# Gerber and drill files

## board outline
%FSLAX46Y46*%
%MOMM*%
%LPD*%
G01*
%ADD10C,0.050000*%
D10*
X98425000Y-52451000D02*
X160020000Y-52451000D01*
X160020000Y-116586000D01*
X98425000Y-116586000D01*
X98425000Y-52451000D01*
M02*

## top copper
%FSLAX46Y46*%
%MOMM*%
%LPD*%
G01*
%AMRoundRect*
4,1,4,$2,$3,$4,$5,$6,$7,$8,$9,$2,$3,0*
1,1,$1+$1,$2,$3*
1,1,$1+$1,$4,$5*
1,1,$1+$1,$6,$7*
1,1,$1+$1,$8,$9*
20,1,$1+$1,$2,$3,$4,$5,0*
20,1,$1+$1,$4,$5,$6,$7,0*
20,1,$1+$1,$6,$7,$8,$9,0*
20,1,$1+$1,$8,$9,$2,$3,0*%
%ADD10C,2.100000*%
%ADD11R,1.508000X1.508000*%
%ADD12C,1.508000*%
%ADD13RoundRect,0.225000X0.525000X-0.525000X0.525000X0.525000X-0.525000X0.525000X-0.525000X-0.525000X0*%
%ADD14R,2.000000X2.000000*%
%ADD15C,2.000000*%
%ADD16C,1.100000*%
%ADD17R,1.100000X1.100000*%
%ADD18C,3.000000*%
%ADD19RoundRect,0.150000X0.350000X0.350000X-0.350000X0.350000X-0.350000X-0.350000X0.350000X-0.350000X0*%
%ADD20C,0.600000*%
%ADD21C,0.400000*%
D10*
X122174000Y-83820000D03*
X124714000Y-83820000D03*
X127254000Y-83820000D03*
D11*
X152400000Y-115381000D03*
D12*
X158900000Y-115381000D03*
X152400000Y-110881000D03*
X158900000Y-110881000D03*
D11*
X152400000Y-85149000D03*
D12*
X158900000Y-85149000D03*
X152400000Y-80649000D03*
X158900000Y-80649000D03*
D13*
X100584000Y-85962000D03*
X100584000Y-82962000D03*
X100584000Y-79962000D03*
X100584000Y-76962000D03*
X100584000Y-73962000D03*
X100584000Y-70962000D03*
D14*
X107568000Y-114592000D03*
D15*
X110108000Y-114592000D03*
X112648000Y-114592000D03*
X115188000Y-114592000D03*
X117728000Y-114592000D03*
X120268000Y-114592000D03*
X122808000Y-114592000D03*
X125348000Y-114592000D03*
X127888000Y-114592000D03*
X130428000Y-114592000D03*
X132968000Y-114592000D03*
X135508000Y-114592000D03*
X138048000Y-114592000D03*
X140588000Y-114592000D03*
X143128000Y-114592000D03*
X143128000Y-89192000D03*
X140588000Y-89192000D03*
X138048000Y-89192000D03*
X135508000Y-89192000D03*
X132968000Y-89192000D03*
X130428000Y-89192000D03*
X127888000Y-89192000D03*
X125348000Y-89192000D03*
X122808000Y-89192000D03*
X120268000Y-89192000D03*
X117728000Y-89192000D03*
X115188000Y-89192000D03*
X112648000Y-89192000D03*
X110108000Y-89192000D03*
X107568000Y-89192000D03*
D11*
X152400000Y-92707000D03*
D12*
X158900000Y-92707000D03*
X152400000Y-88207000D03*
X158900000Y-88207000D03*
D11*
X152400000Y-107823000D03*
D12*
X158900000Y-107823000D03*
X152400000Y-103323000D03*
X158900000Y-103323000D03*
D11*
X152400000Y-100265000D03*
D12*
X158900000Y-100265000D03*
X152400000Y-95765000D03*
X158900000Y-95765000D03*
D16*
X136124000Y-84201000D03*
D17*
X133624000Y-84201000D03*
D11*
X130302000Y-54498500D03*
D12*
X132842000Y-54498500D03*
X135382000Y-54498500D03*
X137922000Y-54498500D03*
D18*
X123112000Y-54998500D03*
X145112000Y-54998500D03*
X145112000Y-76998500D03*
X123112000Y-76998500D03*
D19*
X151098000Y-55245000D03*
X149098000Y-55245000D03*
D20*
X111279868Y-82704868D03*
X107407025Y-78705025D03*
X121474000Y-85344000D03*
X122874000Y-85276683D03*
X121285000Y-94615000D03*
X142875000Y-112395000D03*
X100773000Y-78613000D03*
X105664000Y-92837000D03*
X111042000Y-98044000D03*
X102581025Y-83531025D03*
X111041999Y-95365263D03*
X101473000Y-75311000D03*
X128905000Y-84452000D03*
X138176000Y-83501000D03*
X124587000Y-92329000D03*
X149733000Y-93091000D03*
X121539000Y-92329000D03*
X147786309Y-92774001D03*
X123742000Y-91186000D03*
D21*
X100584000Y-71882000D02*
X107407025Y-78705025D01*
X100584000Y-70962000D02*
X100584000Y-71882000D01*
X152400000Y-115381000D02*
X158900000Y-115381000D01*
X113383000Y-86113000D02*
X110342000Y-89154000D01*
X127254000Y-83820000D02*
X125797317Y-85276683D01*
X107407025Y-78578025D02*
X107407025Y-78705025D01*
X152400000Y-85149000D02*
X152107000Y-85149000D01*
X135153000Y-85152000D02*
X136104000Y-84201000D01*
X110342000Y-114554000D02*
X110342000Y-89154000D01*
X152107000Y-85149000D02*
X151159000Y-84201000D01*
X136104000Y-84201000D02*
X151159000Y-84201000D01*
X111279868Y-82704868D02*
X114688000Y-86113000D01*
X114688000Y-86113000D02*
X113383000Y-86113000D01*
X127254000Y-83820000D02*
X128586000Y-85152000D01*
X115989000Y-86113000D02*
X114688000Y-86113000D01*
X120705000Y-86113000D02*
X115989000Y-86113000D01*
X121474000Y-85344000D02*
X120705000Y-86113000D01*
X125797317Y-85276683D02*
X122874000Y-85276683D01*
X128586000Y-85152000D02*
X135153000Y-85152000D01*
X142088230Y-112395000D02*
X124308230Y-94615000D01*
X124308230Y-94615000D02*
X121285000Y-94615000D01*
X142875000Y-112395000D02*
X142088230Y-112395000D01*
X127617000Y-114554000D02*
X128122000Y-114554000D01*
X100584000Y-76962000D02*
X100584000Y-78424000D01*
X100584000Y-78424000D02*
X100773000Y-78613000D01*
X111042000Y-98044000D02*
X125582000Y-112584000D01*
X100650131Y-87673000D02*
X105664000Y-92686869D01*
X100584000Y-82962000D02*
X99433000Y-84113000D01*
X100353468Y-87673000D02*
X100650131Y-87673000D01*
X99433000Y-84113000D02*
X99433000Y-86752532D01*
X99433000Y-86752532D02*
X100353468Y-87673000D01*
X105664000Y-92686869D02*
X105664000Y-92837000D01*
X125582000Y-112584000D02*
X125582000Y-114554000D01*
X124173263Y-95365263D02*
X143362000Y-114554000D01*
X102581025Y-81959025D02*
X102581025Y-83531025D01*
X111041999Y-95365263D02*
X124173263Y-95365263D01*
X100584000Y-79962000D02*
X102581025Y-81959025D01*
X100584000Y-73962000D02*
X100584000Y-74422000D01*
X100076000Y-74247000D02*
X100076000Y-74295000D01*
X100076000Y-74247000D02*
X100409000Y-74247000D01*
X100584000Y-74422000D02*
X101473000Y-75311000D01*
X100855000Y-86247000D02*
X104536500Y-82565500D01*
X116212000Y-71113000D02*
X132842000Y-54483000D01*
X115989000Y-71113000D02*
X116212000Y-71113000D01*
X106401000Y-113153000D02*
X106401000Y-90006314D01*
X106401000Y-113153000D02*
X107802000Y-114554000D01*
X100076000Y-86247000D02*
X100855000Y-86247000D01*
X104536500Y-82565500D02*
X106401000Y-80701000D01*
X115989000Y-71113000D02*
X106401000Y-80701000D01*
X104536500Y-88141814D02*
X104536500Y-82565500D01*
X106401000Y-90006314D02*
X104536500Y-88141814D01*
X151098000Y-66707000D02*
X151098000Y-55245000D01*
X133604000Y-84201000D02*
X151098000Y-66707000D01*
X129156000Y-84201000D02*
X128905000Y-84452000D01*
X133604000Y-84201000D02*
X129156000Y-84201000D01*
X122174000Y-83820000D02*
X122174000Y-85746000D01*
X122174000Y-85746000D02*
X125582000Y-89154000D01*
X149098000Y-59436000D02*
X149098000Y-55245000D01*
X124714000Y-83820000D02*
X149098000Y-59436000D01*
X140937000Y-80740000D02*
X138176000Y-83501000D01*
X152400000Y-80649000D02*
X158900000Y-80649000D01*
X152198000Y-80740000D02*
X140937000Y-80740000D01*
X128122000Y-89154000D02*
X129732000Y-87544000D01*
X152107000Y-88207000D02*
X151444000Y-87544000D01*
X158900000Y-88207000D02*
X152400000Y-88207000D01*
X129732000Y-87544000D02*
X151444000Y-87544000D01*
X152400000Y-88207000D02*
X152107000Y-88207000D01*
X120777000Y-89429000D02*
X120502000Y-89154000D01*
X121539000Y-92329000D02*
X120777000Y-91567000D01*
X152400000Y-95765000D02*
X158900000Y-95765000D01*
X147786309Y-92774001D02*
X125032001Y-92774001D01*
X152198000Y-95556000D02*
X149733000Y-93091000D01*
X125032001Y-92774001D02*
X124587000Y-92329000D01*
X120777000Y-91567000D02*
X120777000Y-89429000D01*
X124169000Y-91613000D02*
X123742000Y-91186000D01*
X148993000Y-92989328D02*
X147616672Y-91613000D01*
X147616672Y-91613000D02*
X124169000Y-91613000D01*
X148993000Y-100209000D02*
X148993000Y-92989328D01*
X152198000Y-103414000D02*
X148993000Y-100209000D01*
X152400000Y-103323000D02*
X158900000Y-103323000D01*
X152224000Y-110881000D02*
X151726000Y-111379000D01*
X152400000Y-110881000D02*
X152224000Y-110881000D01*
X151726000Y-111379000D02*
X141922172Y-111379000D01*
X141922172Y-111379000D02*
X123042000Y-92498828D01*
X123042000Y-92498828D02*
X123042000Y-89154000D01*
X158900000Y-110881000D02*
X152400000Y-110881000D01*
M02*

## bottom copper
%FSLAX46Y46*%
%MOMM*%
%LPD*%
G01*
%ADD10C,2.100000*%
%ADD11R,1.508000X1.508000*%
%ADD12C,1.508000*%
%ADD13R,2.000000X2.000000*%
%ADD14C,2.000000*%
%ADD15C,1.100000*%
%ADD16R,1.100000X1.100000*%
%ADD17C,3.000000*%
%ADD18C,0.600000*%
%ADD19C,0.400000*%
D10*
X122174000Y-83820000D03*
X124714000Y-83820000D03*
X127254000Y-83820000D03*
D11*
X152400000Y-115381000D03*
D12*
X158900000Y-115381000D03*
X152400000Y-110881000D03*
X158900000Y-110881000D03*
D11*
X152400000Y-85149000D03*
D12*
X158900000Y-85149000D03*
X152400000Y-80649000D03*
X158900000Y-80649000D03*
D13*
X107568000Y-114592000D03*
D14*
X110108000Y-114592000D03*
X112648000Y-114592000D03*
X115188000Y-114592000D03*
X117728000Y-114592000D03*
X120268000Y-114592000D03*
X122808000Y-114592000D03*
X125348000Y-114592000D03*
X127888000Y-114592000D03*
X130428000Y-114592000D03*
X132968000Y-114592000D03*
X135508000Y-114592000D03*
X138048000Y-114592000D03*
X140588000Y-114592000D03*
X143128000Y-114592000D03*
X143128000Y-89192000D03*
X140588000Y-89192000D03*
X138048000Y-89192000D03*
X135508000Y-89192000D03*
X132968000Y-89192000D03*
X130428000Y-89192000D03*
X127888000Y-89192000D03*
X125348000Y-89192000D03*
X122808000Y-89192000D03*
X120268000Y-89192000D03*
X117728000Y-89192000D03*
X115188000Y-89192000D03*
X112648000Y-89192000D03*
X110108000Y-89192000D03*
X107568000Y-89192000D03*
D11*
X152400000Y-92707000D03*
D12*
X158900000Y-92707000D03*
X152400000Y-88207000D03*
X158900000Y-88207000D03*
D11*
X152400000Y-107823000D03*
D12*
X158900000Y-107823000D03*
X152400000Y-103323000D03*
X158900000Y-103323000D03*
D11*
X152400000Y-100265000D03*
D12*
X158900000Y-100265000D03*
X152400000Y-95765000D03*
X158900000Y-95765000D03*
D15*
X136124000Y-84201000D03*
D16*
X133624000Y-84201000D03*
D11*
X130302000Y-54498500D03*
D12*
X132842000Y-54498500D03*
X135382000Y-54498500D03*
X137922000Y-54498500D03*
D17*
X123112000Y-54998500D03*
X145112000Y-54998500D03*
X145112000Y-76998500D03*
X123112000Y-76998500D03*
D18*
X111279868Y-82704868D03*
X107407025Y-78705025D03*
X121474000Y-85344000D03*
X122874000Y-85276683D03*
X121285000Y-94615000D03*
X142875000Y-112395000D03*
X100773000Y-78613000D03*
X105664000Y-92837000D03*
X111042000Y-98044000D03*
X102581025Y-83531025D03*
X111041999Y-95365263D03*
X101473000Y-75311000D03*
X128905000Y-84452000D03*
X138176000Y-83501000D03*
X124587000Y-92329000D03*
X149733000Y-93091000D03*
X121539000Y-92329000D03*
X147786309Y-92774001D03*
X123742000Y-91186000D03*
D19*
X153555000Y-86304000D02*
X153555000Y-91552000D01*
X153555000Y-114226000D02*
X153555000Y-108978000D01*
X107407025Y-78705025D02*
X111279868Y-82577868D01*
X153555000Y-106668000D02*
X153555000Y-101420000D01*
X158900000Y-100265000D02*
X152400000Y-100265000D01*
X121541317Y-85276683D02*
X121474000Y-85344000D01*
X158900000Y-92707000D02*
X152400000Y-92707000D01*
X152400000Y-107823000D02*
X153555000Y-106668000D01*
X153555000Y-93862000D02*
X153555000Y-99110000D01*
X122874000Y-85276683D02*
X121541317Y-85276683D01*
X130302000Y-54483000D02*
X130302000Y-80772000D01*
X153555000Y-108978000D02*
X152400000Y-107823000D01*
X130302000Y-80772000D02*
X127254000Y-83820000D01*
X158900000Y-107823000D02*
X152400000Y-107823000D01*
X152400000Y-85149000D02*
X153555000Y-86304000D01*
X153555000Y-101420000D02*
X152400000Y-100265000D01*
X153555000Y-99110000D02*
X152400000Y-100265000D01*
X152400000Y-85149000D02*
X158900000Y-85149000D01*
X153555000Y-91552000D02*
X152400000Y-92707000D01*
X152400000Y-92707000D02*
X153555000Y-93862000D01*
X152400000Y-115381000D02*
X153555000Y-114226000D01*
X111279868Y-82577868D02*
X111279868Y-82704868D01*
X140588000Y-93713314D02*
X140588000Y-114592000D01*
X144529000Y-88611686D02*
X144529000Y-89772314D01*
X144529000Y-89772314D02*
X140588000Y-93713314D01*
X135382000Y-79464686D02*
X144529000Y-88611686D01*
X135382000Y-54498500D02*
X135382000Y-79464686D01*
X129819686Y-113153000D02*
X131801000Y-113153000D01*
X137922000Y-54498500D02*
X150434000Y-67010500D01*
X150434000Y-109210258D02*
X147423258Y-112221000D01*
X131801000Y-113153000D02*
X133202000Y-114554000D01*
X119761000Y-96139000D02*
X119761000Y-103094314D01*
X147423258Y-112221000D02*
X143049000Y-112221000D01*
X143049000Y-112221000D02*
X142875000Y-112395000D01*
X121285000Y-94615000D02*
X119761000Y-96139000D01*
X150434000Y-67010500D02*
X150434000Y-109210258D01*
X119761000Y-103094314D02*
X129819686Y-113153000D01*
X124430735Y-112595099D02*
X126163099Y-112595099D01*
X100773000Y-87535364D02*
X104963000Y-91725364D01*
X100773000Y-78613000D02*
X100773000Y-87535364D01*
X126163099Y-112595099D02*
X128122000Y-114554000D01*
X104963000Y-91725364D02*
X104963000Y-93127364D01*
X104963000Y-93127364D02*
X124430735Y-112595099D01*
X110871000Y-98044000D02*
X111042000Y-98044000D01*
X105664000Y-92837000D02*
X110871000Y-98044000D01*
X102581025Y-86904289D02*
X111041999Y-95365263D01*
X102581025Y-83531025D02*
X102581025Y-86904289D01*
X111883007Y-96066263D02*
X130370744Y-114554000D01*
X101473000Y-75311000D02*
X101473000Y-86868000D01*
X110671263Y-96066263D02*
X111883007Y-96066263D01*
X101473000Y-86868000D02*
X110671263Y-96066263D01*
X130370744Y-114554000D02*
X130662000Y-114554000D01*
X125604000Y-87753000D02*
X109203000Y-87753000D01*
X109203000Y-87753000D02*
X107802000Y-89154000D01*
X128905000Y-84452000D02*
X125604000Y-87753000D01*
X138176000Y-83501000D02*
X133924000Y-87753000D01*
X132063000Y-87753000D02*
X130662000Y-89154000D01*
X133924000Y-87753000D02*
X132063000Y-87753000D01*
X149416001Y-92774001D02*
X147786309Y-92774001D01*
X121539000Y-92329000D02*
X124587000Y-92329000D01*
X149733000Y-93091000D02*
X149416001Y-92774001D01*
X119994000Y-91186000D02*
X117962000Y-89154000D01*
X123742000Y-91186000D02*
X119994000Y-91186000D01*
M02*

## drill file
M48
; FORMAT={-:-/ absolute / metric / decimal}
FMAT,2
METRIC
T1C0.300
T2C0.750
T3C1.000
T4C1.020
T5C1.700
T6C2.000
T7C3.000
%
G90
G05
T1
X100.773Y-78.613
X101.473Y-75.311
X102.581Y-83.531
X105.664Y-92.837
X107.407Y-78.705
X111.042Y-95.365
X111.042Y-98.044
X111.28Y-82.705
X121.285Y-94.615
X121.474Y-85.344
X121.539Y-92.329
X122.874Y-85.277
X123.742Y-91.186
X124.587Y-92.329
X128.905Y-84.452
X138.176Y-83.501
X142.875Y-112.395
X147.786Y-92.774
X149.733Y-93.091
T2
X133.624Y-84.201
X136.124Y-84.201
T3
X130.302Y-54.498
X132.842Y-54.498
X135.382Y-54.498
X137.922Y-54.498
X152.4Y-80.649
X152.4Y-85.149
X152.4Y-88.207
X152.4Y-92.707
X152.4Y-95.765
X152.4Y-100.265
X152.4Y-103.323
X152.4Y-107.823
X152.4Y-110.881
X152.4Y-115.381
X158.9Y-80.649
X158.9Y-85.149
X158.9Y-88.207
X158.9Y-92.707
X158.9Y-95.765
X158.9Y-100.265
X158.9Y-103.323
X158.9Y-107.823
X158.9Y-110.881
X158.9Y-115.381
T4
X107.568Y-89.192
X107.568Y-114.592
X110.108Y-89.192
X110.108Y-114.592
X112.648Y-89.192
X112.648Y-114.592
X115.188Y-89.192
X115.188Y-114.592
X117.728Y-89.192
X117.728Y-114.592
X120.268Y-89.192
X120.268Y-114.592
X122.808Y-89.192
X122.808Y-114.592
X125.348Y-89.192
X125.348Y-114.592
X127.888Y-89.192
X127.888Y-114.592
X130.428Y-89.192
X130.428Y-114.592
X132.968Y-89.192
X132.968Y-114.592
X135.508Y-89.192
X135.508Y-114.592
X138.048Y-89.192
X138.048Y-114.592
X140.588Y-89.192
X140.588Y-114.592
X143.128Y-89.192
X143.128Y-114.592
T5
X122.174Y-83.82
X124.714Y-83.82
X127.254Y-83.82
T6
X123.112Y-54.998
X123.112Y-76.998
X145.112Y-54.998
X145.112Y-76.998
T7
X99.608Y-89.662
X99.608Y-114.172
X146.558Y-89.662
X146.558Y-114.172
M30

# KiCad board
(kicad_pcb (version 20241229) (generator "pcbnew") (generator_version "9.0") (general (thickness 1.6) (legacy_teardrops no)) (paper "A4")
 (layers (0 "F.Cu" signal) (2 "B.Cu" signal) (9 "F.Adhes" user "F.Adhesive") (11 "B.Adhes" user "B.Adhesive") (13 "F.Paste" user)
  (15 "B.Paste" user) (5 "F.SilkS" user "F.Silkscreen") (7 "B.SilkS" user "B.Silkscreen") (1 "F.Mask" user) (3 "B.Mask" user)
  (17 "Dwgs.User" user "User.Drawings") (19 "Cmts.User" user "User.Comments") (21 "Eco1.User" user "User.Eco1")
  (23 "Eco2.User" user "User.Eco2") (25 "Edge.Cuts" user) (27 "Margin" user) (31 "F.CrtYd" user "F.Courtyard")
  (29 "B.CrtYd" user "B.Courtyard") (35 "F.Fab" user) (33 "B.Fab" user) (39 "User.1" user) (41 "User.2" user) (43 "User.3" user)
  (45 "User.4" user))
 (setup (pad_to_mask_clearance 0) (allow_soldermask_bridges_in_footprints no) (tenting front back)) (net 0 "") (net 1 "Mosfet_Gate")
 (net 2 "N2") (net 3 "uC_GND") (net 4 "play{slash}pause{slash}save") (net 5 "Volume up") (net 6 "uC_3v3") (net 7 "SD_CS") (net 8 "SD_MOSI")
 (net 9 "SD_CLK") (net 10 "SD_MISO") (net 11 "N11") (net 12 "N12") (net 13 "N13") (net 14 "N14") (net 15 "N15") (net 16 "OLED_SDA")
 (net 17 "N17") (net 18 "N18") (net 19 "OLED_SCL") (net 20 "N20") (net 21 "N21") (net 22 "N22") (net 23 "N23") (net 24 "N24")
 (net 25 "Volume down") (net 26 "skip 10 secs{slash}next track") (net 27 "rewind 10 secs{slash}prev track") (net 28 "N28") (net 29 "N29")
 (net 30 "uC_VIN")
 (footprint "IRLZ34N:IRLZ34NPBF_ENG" (layer "F.Cu") (at 124.714 83.82)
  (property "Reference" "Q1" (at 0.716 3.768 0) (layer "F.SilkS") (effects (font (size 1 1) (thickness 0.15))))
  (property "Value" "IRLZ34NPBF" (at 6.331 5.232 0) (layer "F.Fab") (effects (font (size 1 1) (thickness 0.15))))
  (pad "1" thru_hole circle (at -2.54 0) (size 2.1 2.1) (drill 1.7) (layers "*.Cu" "*.Mask") (remove_unused_layers no) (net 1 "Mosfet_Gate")
   (solder_mask_margin 0.102))
  (pad "2" thru_hole circle (at 0 0) (size 2.1 2.1) (drill 1.7) (layers "*.Cu" "*.Mask") (remove_unused_layers no) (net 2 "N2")
   (solder_mask_margin 0.102))
  (pad "3" thru_hole circle (at 2.54 0) (size 2.1 2.1) (drill 1.7) (layers "*.Cu" "*.Mask") (remove_unused_layers no) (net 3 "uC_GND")
   (solder_mask_margin 0.102)))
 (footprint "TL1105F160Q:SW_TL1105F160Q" (layer "F.Cu") (at 155.65 113.131)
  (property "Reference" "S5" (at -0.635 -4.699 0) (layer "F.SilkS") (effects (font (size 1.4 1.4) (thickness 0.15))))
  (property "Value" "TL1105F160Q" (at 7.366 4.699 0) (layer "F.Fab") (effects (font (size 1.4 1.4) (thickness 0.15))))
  (pad "1" thru_hole rect (at -3.25 2.25) (size 1.508 1.508) (drill 1) (layers "*.Cu" "*.Mask") (remove_unused_layers no) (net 3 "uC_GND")
   (solder_mask_margin 0.102))
  (pad "2" thru_hole circle (at 3.25 2.25) (size 1.508 1.508) (drill 1) (layers "*.Cu" "*.Mask") (remove_unused_layers no) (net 3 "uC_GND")
   (solder_mask_margin 0.102))
  (pad "3" thru_hole circle (at -3.25 -2.25) (size 1.508 1.508) (drill 1) (layers "*.Cu" "*.Mask") (remove_unused_layers no)
   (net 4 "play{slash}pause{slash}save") (solder_mask_margin 0.102))
  (pad "4" thru_hole circle (at 3.25 -2.25) (size 1.508 1.508) (drill 1) (layers "*.Cu" "*.Mask") (remove_unused_layers no)
   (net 4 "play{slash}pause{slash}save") (solder_mask_margin 0.102)))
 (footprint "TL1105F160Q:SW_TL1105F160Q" (layer "F.Cu") (at 155.65 82.899)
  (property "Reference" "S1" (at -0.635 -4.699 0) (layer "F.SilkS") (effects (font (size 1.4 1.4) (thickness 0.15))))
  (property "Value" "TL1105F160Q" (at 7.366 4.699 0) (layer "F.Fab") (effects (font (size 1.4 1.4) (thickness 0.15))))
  (pad "1" thru_hole rect (at -3.25 2.25) (size 1.508 1.508) (drill 1) (layers "*.Cu" "*.Mask") (remove_unused_layers no) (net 3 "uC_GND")
   (solder_mask_margin 0.102))
  (pad "2" thru_hole circle (at 3.25 2.25) (size 1.508 1.508) (drill 1) (layers "*.Cu" "*.Mask") (remove_unused_layers no) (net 3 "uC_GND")
   (solder_mask_margin 0.102))
  (pad "3" thru_hole circle (at -3.25 -2.25) (size 1.508 1.508) (drill 1) (layers "*.Cu" "*.Mask") (remove_unused_layers no)
   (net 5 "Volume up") (solder_mask_margin 0.102))
  (pad "4" thru_hole circle (at 3.25 -2.25) (size 1.508 1.508) (drill 1) (layers "*.Cu" "*.Mask") (remove_unused_layers no)
   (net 5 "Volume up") (solder_mask_margin 0.102)))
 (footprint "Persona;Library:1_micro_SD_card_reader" (layer "F.Cu") (at 97.334 78.962 90)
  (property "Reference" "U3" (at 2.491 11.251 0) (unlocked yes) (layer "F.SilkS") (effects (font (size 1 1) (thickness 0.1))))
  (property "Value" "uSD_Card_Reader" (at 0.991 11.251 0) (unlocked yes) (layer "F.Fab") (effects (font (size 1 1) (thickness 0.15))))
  (pad "1" smd roundrect (at -7 3.25 90) (size 1.5 1.5) (layers "F.Cu" "F.Mask" "F.Paste") (roundrect_rratio 0.15) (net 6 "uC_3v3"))
  (pad "2" smd roundrect (at -4 3.25 90) (size 1.5 1.5) (layers "F.Cu" "F.Mask" "F.Paste") (roundrect_rratio 0.15) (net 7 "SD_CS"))
  (pad "3" smd roundrect (at -1 3.25 90) (size 1.5 1.5) (layers "F.Cu" "F.Mask" "F.Paste") (roundrect_rratio 0.15) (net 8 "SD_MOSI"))
  (pad "4" smd roundrect (at 2 3.25 90) (size 1.5 1.5) (layers "F.Cu" "F.Mask" "F.Paste") (roundrect_rratio 0.15) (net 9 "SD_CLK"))
  (pad "5" smd roundrect (at 5 3.25 90) (size 1.5 1.5) (layers "F.Cu" "F.Mask" "F.Paste") (roundrect_rratio 0.15) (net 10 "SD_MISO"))
  (pad "6" smd roundrect (at 8 3.25 90) (size 1.5 1.5) (layers "F.Cu" "F.Mask" "F.Paste") (roundrect_rratio 0.15) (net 3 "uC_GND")))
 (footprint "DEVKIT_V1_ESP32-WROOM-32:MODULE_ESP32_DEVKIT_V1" (layer "F.Cu") (at 123.083 101.892 90)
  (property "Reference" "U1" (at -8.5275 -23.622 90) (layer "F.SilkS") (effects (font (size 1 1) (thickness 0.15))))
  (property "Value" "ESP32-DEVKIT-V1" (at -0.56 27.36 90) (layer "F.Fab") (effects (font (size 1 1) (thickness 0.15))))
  (pad "" np_thru_hole circle (at -12.28 -23.475 90) (size 3 3) (drill 3) (layers "*.Cu" "*.Mask"))
  (pad "" np_thru_hole circle (at -12.28 23.475 90) (size 3 3) (drill 3) (layers "*.Cu" "*.Mask"))
  (pad "" np_thru_hole circle (at 12.23 -23.475 90) (size 3 3) (drill 3) (layers "*.Cu" "*.Mask"))
  (pad "" np_thru_hole circle (at 12.23 23.475 90) (size 3 3) (drill 3) (layers "*.Cu" "*.Mask"))
  (pad "1" thru_hole rect (at -12.7 -15.515 90) (size 2 2) (drill 1.02) (layers "*.Cu" "*.Mask") (remove_unused_layers no) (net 6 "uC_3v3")
   (solder_mask_margin 0.102))
  (pad "2" thru_hole circle (at -12.7 -12.975 90) (size 2 2) (drill 1.02) (layers "*.Cu" "*.Mask") (remove_unused_layers no)
   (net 3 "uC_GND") (solder_mask_margin 0.102))
  (pad "3" thru_hole circle (at -12.7 -10.435 90) (size 2 2) (drill 1.02) (layers "*.Cu" "*.Mask") (remove_unused_layers no) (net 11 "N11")
   (solder_mask_margin 0.102))
  (pad "4" thru_hole circle (at -12.7 -7.895 90) (size 2 2) (drill 1.02) (layers "*.Cu" "*.Mask") (remove_unused_layers no) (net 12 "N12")
   (solder_mask_margin 0.102))
  (pad "5" thru_hole circle (at -12.7 -5.355 90) (size 2 2) (drill 1.02) (layers "*.Cu" "*.Mask") (remove_unused_layers no) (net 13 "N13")
   (solder_mask_margin 0.102))
  (pad "6" thru_hole circle (at -12.7 -2.815 90) (size 2 2) (drill 1.02) (layers "*.Cu" "*.Mask") (remove_unused_layers no) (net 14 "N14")
   (solder_mask_margin 0.102))
  (pad "7" thru_hole circle (at -12.7 -0.275 90) (size 2 2) (drill 1.02) (layers "*.Cu" "*.Mask") (remove_unused_layers no) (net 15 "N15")
   (solder_mask_margin 0.102))
  (pad "8" thru_hole circle (at -12.7 2.265 90) (size 2 2) (drill 1.02) (layers "*.Cu" "*.Mask") (remove_unused_layers no) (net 7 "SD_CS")
   (solder_mask_margin 0.102))
  (pad "9" thru_hole circle (at -12.7 4.805 90) (size 2 2) (drill 1.02) (layers "*.Cu" "*.Mask") (remove_unused_layers no) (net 9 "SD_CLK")
   (solder_mask_margin 0.102))
  (pad "10" thru_hole circle (at -12.7 7.345 90) (size 2 2) (drill 1.02) (layers "*.Cu" "*.Mask") (remove_unused_layers no)
   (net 10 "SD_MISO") (solder_mask_margin 0.102))
  (pad "11" thru_hole circle (at -12.7 9.885 90) (size 2 2) (drill 1.02) (layers "*.Cu" "*.Mask") (remove_unused_layers no)
   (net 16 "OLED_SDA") (solder_mask_margin 0.102))
  (pad "12" thru_hole circle (at -12.7 12.425 90) (size 2 2) (drill 1.02) (layers "*.Cu" "*.Mask") (remove_unused_layers no) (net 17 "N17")
   (solder_mask_margin 0.102))
  (pad "13" thru_hole circle (at -12.7 14.965 90) (size 2 2) (drill 1.02) (layers "*.Cu" "*.Mask") (remove_unused_layers no) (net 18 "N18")
   (solder_mask_margin 0.102))
  (pad "14" thru_hole circle (at -12.7 17.505 90) (size 2 2) (drill 1.02) (layers "*.Cu" "*.Mask") (remove_unused_layers no)
   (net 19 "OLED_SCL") (solder_mask_margin 0.102))
  (pad "15" thru_hole circle (at -12.7 20.045 90) (size 2 2) (drill 1.02) (layers "*.Cu" "*.Mask") (remove_unused_layers no)
   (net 8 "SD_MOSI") (solder_mask_margin 0.102))
  (pad "16" thru_hole circle (at 12.7 20.045 90) (size 2 2) (drill 1.02) (layers "*.Cu" "*.Mask") (remove_unused_layers no) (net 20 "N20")
   (solder_mask_margin 0.102))
  (pad "17" thru_hole circle (at 12.7 17.505 90) (size 2 2) (drill 1.02) (layers "*.Cu" "*.Mask") (remove_unused_layers no) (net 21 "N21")
   (solder_mask_margin 0.102))
  (pad "18" thru_hole circle (at 12.7 14.965 90) (size 2 2) (drill 1.02) (layers "*.Cu" "*.Mask") (remove_unused_layers no) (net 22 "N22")
   (solder_mask_margin 0.102))
  (pad "19" thru_hole circle (at 12.7 12.425 90) (size 2 2) (drill 1.02) (layers "*.Cu" "*.Mask") (remove_unused_layers no) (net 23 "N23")
   (solder_mask_margin 0.102))
  (pad "20" thru_hole circle (at 12.7 9.885 90) (size 2 2) (drill 1.02) (layers "*.Cu" "*.Mask") (remove_unused_layers no) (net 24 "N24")
   (solder_mask_margin 0.102))
  (pad "21" thru_hole circle (at 12.7 7.345 90) (size 2 2) (drill 1.02) (layers "*.Cu" "*.Mask") (remove_unused_layers no)
   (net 5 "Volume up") (solder_mask_margin 0.102))
  (pad "22" thru_hole circle (at 12.7 4.805 90) (size 2 2) (drill 1.02) (layers "*.Cu" "*.Mask") (remove_unused_layers no)
   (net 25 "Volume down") (solder_mask_margin 0.102))
  (pad "23" thru_hole circle (at 12.7 2.265 90) (size 2 2) (drill 1.02) (layers "*.Cu" "*.Mask") (remove_unused_layers no)
   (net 1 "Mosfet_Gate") (solder_mask_margin 0.102))
  (pad "24" thru_hole circle (at 12.7 -0.275 90) (size 2 2) (drill 1.02) (layers "*.Cu" "*.Mask") (remove_unused_layers no)
   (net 4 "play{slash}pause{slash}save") (solder_mask_margin 0.102))
  (pad "25" thru_hole circle (at 12.7 -2.815 90) (size 2 2) (drill 1.02) (layers "*.Cu" "*.Mask") (remove_unused_layers no)
   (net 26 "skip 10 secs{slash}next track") (solder_mask_margin 0.102))
  (pad "26" thru_hole circle (at 12.7 -5.355 90) (size 2 2) (drill 1.02) (layers "*.Cu" "*.Mask") (remove_unused_layers no)
   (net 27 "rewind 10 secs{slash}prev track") (solder_mask_margin 0.102))
  (pad "27" thru_hole circle (at 12.7 -7.895 90) (size 2 2) (drill 1.02) (layers "*.Cu" "*.Mask") (remove_unused_layers no) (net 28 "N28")
   (solder_mask_margin 0.102))
  (pad "28" thru_hole circle (at 12.7 -10.435 90) (size 2 2) (drill 1.02) (layers "*.Cu" "*.Mask") (remove_unused_layers no) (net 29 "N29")
   (solder_mask_margin 0.102))
  (pad "29" thru_hole circle (at 12.7 -12.975 90) (size 2 2) (drill 1.02) (layers "*.Cu" "*.Mask") (remove_unused_layers no)
   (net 3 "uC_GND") (solder_mask_margin 0.102))
  (pad "30" thru_hole circle (at 12.7 -15.515 90) (size 2 2) (drill 1.02) (layers "*.Cu" "*.Mask") (remove_unused_layers no)
   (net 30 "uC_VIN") (solder_mask_margin 0.102))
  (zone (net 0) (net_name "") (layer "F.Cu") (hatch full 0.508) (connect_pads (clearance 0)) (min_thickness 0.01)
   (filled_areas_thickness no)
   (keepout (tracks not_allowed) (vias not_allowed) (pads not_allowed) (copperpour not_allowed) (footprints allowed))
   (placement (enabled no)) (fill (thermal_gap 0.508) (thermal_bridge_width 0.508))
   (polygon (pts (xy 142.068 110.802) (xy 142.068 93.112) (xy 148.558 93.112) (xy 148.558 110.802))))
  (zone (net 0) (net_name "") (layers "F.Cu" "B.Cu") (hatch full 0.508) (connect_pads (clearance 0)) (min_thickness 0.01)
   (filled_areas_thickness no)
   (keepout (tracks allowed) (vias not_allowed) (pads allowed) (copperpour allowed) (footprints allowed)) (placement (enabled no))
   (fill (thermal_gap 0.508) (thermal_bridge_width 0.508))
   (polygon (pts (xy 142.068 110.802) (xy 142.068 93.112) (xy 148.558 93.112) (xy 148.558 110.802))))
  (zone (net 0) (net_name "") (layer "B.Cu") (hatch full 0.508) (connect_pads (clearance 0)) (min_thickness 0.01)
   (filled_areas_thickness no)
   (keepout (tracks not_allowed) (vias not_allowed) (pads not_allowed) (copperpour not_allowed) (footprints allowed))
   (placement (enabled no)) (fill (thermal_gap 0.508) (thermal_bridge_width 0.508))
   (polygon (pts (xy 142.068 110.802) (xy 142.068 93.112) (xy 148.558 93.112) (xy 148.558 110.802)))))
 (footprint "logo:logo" (layer "F.Cu") (at 155.321 72.009)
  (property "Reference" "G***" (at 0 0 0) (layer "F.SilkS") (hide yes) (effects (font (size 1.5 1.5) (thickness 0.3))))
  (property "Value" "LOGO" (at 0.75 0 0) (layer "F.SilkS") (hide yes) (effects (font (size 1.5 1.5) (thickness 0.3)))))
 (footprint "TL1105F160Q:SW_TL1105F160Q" (layer "F.Cu") (at 155.65 90.457)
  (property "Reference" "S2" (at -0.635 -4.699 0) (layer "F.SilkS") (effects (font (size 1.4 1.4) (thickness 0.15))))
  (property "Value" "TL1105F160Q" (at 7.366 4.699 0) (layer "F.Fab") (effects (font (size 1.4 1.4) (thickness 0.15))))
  (pad "1" thru_hole rect (at -3.25 2.25) (size 1.508 1.508) (drill 1) (layers "*.Cu" "*.Mask") (remove_unused_layers no) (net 3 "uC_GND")
   (solder_mask_margin 0.102))
  (pad "2" thru_hole circle (at 3.25 2.25) (size 1.508 1.508) (drill 1) (layers "*.Cu" "*.Mask") (remove_unused_layers no) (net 3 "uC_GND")
   (solder_mask_margin 0.102))
  (pad "3" thru_hole circle (at -3.25 -2.25) (size 1.508 1.508) (drill 1) (layers "*.Cu" "*.Mask") (remove_unused_layers no)
   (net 25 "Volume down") (solder_mask_margin 0.102))
  (pad "4" thru_hole circle (at 3.25 -2.25) (size 1.508 1.508) (drill 1) (layers "*.Cu" "*.Mask") (remove_unused_layers no)
   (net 25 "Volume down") (solder_mask_margin 0.102)))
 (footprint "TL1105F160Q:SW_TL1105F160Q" (layer "F.Cu") (at 155.65 105.573)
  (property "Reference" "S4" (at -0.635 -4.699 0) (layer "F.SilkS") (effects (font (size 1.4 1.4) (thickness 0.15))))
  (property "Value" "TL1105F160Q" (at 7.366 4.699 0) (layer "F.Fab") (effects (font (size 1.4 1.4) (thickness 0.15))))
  (pad "1" thru_hole rect (at -3.25 2.25) (size 1.508 1.508) (drill 1) (layers "*.Cu" "*.Mask") (remove_unused_layers no) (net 3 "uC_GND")
   (solder_mask_margin 0.102))
  (pad "2" thru_hole circle (at 3.25 2.25) (size 1.508 1.508) (drill 1) (layers "*.Cu" "*.Mask") (remove_unused_layers no) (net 3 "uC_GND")
   (solder_mask_margin 0.102))
  (pad "3" thru_hole circle (at -3.25 -2.25) (size 1.508 1.508) (drill 1) (layers "*.Cu" "*.Mask") (remove_unused_layers no)
   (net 27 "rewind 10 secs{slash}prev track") (solder_mask_margin 0.102))
  (pad "4" thru_hole circle (at 3.25 -2.25) (size 1.508 1.508) (drill 1) (layers "*.Cu" "*.Mask") (remove_unused_layers no)
   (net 27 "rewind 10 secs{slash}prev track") (solder_mask_margin 0.102)))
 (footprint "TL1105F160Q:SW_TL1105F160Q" (layer "F.Cu") (at 155.65 98.015)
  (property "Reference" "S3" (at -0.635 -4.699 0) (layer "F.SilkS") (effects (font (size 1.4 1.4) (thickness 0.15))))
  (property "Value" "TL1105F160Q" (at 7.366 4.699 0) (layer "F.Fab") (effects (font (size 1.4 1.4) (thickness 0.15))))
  (pad "1" thru_hole rect (at -3.25 2.25) (size 1.508 1.508) (drill 1) (layers "*.Cu" "*.Mask") (remove_unused_layers no) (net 3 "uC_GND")
   (solder_mask_margin 0.102))
  (pad "2" thru_hole circle (at 3.25 2.25) (size 1.508 1.508) (drill 1) (layers "*.Cu" "*.Mask") (remove_unused_layers no) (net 3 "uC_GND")
   (solder_mask_margin 0.102))
  (pad "3" thru_hole circle (at -3.25 -2.25) (size 1.508 1.508) (drill 1) (layers "*.Cu" "*.Mask") (remove_unused_layers no)
   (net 26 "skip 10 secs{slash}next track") (solder_mask_margin 0.102))
  (pad "4" thru_hole circle (at 3.25 -2.25) (size 1.508 1.508) (drill 1) (layers "*.Cu" "*.Mask") (remove_unused_layers no)
   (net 26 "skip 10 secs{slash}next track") (solder_mask_margin 0.102)))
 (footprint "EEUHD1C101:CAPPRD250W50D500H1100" (layer "F.Cu") (at 134.874 84.201)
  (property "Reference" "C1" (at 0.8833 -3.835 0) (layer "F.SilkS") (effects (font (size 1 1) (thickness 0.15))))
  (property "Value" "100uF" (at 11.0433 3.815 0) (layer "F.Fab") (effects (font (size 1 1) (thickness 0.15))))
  (pad "N" thru_hole circle (at 1.25 0) (size 1.1 1.1) (drill 0.75) (layers "*.Cu" "*.Mask") (remove_unused_layers no) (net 3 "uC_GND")
   (solder_mask_margin 0.102))
  (pad "P" thru_hole rect (at -1.25 0) (size 1.1 1.1) (drill 0.75) (layers "*.Cu" "*.Mask") (remove_unused_layers no) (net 30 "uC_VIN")
   (solder_mask_margin 0.102)))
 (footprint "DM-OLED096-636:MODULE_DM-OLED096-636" (layer "F.Cu") (at 134.112 65.9985)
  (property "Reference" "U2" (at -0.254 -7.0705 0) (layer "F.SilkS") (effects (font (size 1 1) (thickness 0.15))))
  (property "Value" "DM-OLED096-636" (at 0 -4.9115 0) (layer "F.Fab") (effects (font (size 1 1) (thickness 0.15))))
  (pad "1" thru_hole rect (at -3.81 -11.5) (size 1.508 1.508) (drill 1) (layers "*.Cu" "*.Mask") (remove_unused_layers no) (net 3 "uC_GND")
   (solder_mask_margin 0.102))
  (pad "2" thru_hole circle (at -1.27 -11.5) (size 1.508 1.508) (drill 1) (layers "*.Cu" "*.Mask") (remove_unused_layers no)
   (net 6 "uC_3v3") (solder_mask_margin 0.102))
  (pad "3" thru_hole circle (at 1.27 -11.5) (size 1.508 1.508) (drill 1) (layers "*.Cu" "*.Mask") (remove_unused_layers no)
   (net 19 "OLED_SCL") (solder_mask_margin 0.102))
  (pad "4" thru_hole circle (at 3.81 -11.5) (size 1.508 1.508) (drill 1) (layers "*.Cu" "*.Mask") (remove_unused_layers no)
   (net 16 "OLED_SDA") (solder_mask_margin 0.102))
  (pad "S1" thru_hole circle (at -11 -11) (size 3 3) (drill 2) (layers "*.Cu" "*.Mask") (remove_unused_layers no) (solder_mask_margin 0.102))
  (pad "S2" thru_hole circle (at 11 -11) (size 3 3) (drill 2) (layers "*.Cu" "*.Mask") (remove_unused_layers no) (solder_mask_margin 0.102))
  (pad "S3" thru_hole circle (at 11 11) (size 3 3) (drill 2) (layers "*.Cu" "*.Mask") (remove_unused_layers no) (solder_mask_margin 0.102))
  (pad "S4" thru_hole circle (at -11 11) (size 3 3) (drill 2) (layers "*.Cu" "*.Mask") (remove_unused_layers no) (solder_mask_margin 0.102)))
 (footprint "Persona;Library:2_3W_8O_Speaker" (layer "F.Cu") (at 150.098 56.245 180)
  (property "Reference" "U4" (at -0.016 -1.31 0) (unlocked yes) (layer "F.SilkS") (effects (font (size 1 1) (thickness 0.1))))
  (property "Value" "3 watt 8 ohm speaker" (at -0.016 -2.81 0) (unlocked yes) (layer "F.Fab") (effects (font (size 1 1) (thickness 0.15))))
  (pad "1" smd roundrect (at -1 1 180) (size 1 1) (layers "F.Cu" "F.Mask" "F.Paste") (roundrect_rratio 0.15) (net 30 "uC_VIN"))
  (pad "2" smd roundrect (at 1 1 180) (size 1 1) (layers "F.Cu" "F.Mask" "F.Paste") (roundrect_rratio 0.15) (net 2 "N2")))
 (gr_rect (start 98.425 52.451) (end 160.02 116.586) (stroke (width 0.05) (type default)) (fill no) (layer "Edge.Cuts"))
 (segment (start 100.584 71.882) (end 107.407025 78.705025) (width 0.4) (layer "F.Cu") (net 3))
 (segment (start 100.584 70.962) (end 100.584 71.882) (width 0.4) (layer "F.Cu") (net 3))
 (segment (start 152.4 115.381) (end 158.9 115.381) (width 0.4) (layer "F.Cu") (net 3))
 (segment (start 113.383 86.113) (end 110.342 89.154) (width 0.4) (layer "F.Cu") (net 3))
 (segment (start 127.254 83.82) (end 125.797317 85.276683) (width 0.4) (layer "F.Cu") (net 3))
 (segment (start 107.407025 78.578025) (end 107.407025 78.705025) (width 0.4) (layer "F.Cu") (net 3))
 (segment (start 152.4 85.149) (end 152.107 85.149) (width 0.4) (layer "F.Cu") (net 3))
 (segment (start 135.153 85.152) (end 136.104 84.201) (width 0.4) (layer "F.Cu") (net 3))
 (segment (start 110.342 114.554) (end 110.342 89.154) (width 0.4) (layer "F.Cu") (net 3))
 (segment (start 152.107 85.149) (end 151.159 84.201) (width 0.4) (layer "F.Cu") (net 3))
 (segment (start 136.104 84.201) (end 151.159 84.201) (width 0.4) (layer "F.Cu") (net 3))
 (segment (start 111.279868 82.704868) (end 114.688 86.113) (width 0.4) (layer "F.Cu") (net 3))
 (segment (start 114.688 86.113) (end 113.383 86.113) (width 0.4) (layer "F.Cu") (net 3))
 (segment (start 127.254 83.82) (end 128.586 85.152) (width 0.4) (layer "F.Cu") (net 3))
 (segment (start 115.989 86.113) (end 114.688 86.113) (width 0.4) (layer "F.Cu") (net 3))
 (segment (start 120.705 86.113) (end 115.989 86.113) (width 0.4) (layer "F.Cu") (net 3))
 (segment (start 121.474 85.344) (end 120.705 86.113) (width 0.4) (layer "F.Cu") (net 3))
 (segment (start 125.797317 85.276683) (end 122.874 85.276683) (width 0.4) (layer "F.Cu") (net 3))
 (segment (start 128.586 85.152) (end 135.153 85.152) (width 0.4) (layer "F.Cu") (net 3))
 (via (at 111.279868 82.704868) (size 0.6) (drill 0.3) (layers "F.Cu" "B.Cu") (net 3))
 (via (at 107.407025 78.705025) (size 0.6) (drill 0.3) (layers "F.Cu" "B.Cu") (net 3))
 (via (at 121.474 85.344) (size 0.6) (drill 0.3) (layers "F.Cu" "B.Cu") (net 3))
 (via (at 122.874 85.276683) (size 0.6) (drill 0.3) (layers "F.Cu" "B.Cu") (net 3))
 (segment (start 153.555 86.304) (end 153.555 91.552) (width 0.4) (layer "B.Cu") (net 3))
 (segment (start 153.555 114.226) (end 153.555 108.978) (width 0.4) (layer "B.Cu") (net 3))
 (segment (start 107.407025 78.705025) (end 111.279868 82.577868) (width 0.4) (layer "B.Cu") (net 3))
 (segment (start 153.555 106.668) (end 153.555 101.42) (width 0.4) (layer "B.Cu") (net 3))
 (segment (start 158.9 100.265) (end 152.4 100.265) (width 0.4) (layer "B.Cu") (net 3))
 (segment (start 121.541317 85.276683) (end 121.474 85.344) (width 0.4) (layer "B.Cu") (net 3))
 (segment (start 158.9 92.707) (end 152.4 92.707) (width 0.4) (layer "B.Cu") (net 3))
 (segment (start 152.4 107.823) (end 153.555 106.668) (width 0.4) (layer "B.Cu") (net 3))
 (segment (start 153.555 93.862) (end 153.555 99.11) (width 0.4) (layer "B.Cu") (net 3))
 (segment (start 122.874 85.276683) (end 121.541317 85.276683) (width 0.4) (layer "B.Cu") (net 3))
 (segment (start 130.302 54.483) (end 130.302 80.772) (width 0.4) (layer "B.Cu") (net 3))
 (segment (start 153.555 108.978) (end 152.4 107.823) (width 0.4) (layer "B.Cu") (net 3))
 (segment (start 130.302 80.772) (end 127.254 83.82) (width 0.4) (layer "B.Cu") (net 3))
 (segment (start 158.9 107.823) (end 152.4 107.823) (width 0.4) (layer "B.Cu") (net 3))
 (segment (start 152.4 85.149) (end 153.555 86.304) (width 0.4) (layer "B.Cu") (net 3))
 (segment (start 153.555 101.42) (end 152.4 100.265) (width 0.4) (layer "B.Cu") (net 3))
 (segment (start 153.555 99.11) (end 152.4 100.265) (width 0.4) (layer "B.Cu") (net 3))
 (segment (start 152.4 85.149) (end 158.9 85.149) (width 0.4) (layer "B.Cu") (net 3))
 (segment (start 153.555 91.552) (end 152.4 92.707) (width 0.4) (layer "B.Cu") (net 3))
 (segment (start 152.4 92.707) (end 153.555 93.862) (width 0.4) (layer "B.Cu") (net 3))
 (segment (start 152.4 115.381) (end 153.555 114.226) (width 0.4) (layer "B.Cu") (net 3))
 (segment (start 111.279868 82.577868) (end 111.279868 82.704868) (width 0.4) (layer "B.Cu") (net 3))
 (segment (start 140.588 93.713314) (end 140.588 114.592) (width 0.4) (layer "B.Cu") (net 19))
 (segment (start 144.529 88.611686) (end 144.529 89.772314) (width 0.4) (layer "B.Cu") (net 19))
 (segment (start 144.529 89.772314) (end 140.588 93.713314) (width 0.4) (layer "B.Cu") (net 19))
 (segment (start 135.382 79.464686) (end 144.529 88.611686) (width 0.4) (layer "B.Cu") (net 19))
 (segment (start 135.382 54.4985) (end 135.382 79.464686) (width 0.4) (layer "B.Cu") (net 19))
 (segment (start 142.08823 112.395) (end 124.30823 94.615) (width 0.4) (layer "F.Cu") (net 16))
 (segment (start 124.30823 94.615) (end 121.285 94.615) (width 0.4) (layer "F.Cu") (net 16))
 (segment (start 142.875 112.395) (end 142.08823 112.395) (width 0.4) (layer "F.Cu") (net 16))
 (via (at 121.285 94.615) (size 0.6) (drill 0.3) (layers "F.Cu" "B.Cu") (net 16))
 (via (at 142.875 112.395) (size 0.6) (drill 0.3) (layers "F.Cu" "B.Cu") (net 16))
 (segment (start 129.819686 113.153) (end 131.801 113.153) (width 0.4) (layer "B.Cu") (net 16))
 (segment (start 137.922 54.4985) (end 150.434 67.0105) (width 0.4) (layer "B.Cu") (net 16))
 (segment (start 150.434 109.210258) (end 147.423258 112.221) (width 0.4) (layer "B.Cu") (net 16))
 (segment (start 131.801 113.153) (end 133.202 114.554) (width 0.4) (layer "B.Cu") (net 16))
 (segment (start 119.761 96.139) (end 119.761 103.094314) (width 0.4) (layer "B.Cu") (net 16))
 (segment (start 147.423258 112.221) (end 143.049 112.221) (width 0.4) (layer "B.Cu") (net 16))
 (segment (start 143.049 112.221) (end 142.875 112.395) (width 0.4) (layer "B.Cu") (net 16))
 (segment (start 121.285 94.615) (end 119.761 96.139) (width 0.4) (layer "B.Cu") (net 16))
 (segment (start 150.434 67.0105) (end 150.434 109.210258) (width 0.4) (layer "B.Cu") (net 16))
 (segment (start 119.761 103.094314) (end 129.819686 113.153) (width 0.4) (layer "B.Cu") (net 16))
 (segment (start 127.617 114.554) (end 128.122 114.554) (width 0.4) (layer "F.Cu") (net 9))
 (segment (start 100.584 76.962) (end 100.584 78.424) (width 0.4) (layer "F.Cu") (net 9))
 (segment (start 100.584 78.424) (end 100.773 78.613) (width 0.4) (layer "F.Cu") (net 9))
 (via (at 100.773 78.613) (size 0.6) (drill 0.3) (layers "F.Cu" "B.Cu") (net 9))
 (segment (start 124.430735 112.595099) (end 126.163099 112.595099) (width 0.4) (layer "B.Cu") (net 9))
 (segment (start 100.773 87.535364) (end 104.963 91.725364) (width 0.4) (layer "B.Cu") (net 9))
 (segment (start 100.773 78.613) (end 100.773 87.535364) (width 0.4) (layer "B.Cu") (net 9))
 (segment (start 126.163099 112.595099) (end 128.122 114.554) (width 0.4) (layer "B.Cu") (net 9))
 (segment (start 104.963 91.725364) (end 104.963 93.127364) (width 0.4) (layer "B.Cu") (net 9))
 (segment (start 104.963 93.127364) (end 124.430735 112.595099) (width 0.4) (layer "B.Cu") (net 9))
 (segment (start 111.042 98.044) (end 125.582 112.584) (width 0.4) (layer "F.Cu") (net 7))
 (segment (start 100.650131 87.673) (end 105.664 92.686869) (width 0.4) (layer "F.Cu") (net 7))
 (segment (start 100.584 82.962) (end 99.433 84.113) (width 0.4) (layer "F.Cu") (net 7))
 (segment (start 100.353468 87.673) (end 100.650131 87.673) (width 0.4) (layer "F.Cu") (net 7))
 (segment (start 99.433 84.113) (end 99.433 86.752532) (width 0.4) (layer "F.Cu") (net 7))
 (segment (start 99.433 86.752532) (end 100.353468 87.673) (width 0.4) (layer "F.Cu") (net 7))
 (segment (start 105.664 92.686869) (end 105.664 92.837) (width 0.4) (layer "F.Cu") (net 7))
 (segment (start 125.582 112.584) (end 125.582 114.554) (width 0.4) (layer "F.Cu") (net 7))
 (via (at 105.664 92.837) (size 0.6) (drill 0.3) (layers "F.Cu" "B.Cu") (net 7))
 (via (at 111.042 98.044) (size 0.6) (drill 0.3) (layers "F.Cu" "B.Cu") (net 7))
 (segment (start 110.871 98.044) (end 111.042 98.044) (width 0.4) (layer "B.Cu") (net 7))
 (segment (start 105.664 92.837) (end 110.871 98.044) (width 0.4) (layer "B.Cu") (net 7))
 (segment (start 124.173263 95.365263) (end 143.362 114.554) (width 0.4) (layer "F.Cu") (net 8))
 (segment (start 102.581025 81.959025) (end 102.581025 83.531025) (width 0.4) (layer "F.Cu") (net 8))
 (segment (start 111.041999 95.365263) (end 124.173263 95.365263) (width 0.4) (layer "F.Cu") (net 8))
 (segment (start 100.584 79.962) (end 102.581025 81.959025) (width 0.4) (layer "F.Cu") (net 8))
 (via (at 102.581025 83.531025) (size 0.6) (drill 0.3) (layers "F.Cu" "B.Cu") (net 8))
 (via (at 111.041999 95.365263) (size 0.6) (drill 0.3) (layers "F.Cu" "B.Cu") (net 8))
 (segment (start 102.581025 86.904289) (end 111.041999 95.365263) (width 0.4) (layer "B.Cu") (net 8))
 (segment (start 102.581025 83.531025) (end 102.581025 86.904289) (width 0.4) (layer "B.Cu") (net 8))
 (segment (start 100.584 73.962) (end 100.584 74.422) (width 0.4) (layer "F.Cu") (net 10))
 (segment (start 100.076 74.247) (end 100.076 74.295) (width 0.4) (layer "F.Cu") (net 10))
 (segment (start 100.076 74.247) (end 100.409 74.247) (width 0.4) (layer "F.Cu") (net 10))
 (segment (start 100.584 74.422) (end 101.473 75.311) (width 0.4) (layer "F.Cu") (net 10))
 (via (at 101.473 75.311) (size 0.6) (drill 0.3) (layers "F.Cu" "B.Cu") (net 10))
 (segment (start 111.883007 96.066263) (end 130.370744 114.554) (width 0.4) (layer "B.Cu") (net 10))
 (segment (start 101.473 75.311) (end 101.473 86.868) (width 0.4) (layer "B.Cu") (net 10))
 (segment (start 110.671263 96.066263) (end 111.883007 96.066263) (width 0.4) (layer "B.Cu") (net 10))
 (segment (start 101.473 86.868) (end 110.671263 96.066263) (width 0.4) (layer "B.Cu") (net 10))
 (segment (start 130.370744 114.554) (end 130.662 114.554) (width 0.4) (layer "B.Cu") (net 10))
 (segment (start 100.855 86.247) (end 104.5365 82.5655) (width 0.4) (layer "F.Cu") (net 6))
 (segment (start 116.212 71.113) (end 132.842 54.483) (width 0.4) (layer "F.Cu") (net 6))
 (segment (start 115.989 71.113) (end 116.212 71.113) (width 0.4) (layer "F.Cu") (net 6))
 (segment (start 106.401 113.153) (end 106.401 90.006314) (width 0.4) (layer "F.Cu") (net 6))
 (segment (start 106.401 113.153) (end 107.802 114.554) (width 0.4) (layer "F.Cu") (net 6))
 (segment (start 100.076 86.247) (end 100.855 86.247) (width 0.4) (layer "F.Cu") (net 6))
 (segment (start 104.5365 82.5655) (end 106.401 80.701) (width 0.4) (layer "F.Cu") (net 6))
 (segment (start 115.989 71.113) (end 106.401 80.701) (width 0.4) (layer "F.Cu") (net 6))
 (segment (start 104.5365 88.141814) (end 104.5365 82.5655) (width 0.4) (layer "F.Cu") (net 6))
 (segment (start 106.401 90.006314) (end 104.5365 88.141814) (width 0.4) (layer "F.Cu") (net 6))
 (segment (start 151.098 66.707) (end 151.098 55.245) (width 0.4) (layer "F.Cu") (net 30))
 (segment (start 133.604 84.201) (end 151.098 66.707) (width 0.4) (layer "F.Cu") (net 30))
 (segment (start 129.156 84.201) (end 128.905 84.452) (width 0.4) (layer "F.Cu") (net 30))
 (segment (start 133.604 84.201) (end 129.156 84.201) (width 0.4) (layer "F.Cu") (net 30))
 (via (at 128.905 84.452) (size 0.6) (drill 0.3) (layers "F.Cu" "B.Cu") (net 30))
 (segment (start 125.604 87.753) (end 109.203 87.753) (width 0.4) (layer "B.Cu") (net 30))
 (segment (start 109.203 87.753) (end 107.802 89.154) (width 0.4) (layer "B.Cu") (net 30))
 (segment (start 128.905 84.452) (end 125.604 87.753) (width 0.4) (layer "B.Cu") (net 30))
 (segment (start 122.174 83.82) (end 122.174 85.746) (width 0.4) (layer "F.Cu") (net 1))
 (segment (start 122.174 85.746) (end 125.582 89.154) (width 0.4) (layer "F.Cu") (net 1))
 (segment (start 149.098 59.436) (end 149.098 55.245) (width 0.4) (layer "F.Cu") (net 2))
 (segment (start 124.714 83.82) (end 149.098 59.436) (width 0.4) (layer "F.Cu") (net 2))
 (segment (start 140.937 80.74) (end 138.176 83.501) (width 0.4) (layer "F.Cu") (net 5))
 (segment (start 152.4 80.649) (end 158.9 80.649) (width 0.4) (layer "F.Cu") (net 5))
 (segment (start 152.198 80.74) (end 140.937 80.74) (width 0.4) (layer "F.Cu") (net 5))
 (via (at 138.176 83.501) (size 0.6) (drill 0.3) (layers "F.Cu" "B.Cu") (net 5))
 (segment (start 138.176 83.501) (end 133.924 87.753) (width 0.4) (layer "B.Cu") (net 5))
 (segment (start 132.063 87.753) (end 130.662 89.154) (width 0.4) (layer "B.Cu") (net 5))
 (segment (start 133.924 87.753) (end 132.063 87.753) (width 0.4) (layer "B.Cu") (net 5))
 (segment (start 128.122 89.154) (end 129.732 87.544) (width 0.4) (layer "F.Cu") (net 25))
 (segment (start 152.107 88.207) (end 151.444 87.544) (width 0.4) (layer "F.Cu") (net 25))
 (segment (start 158.9 88.207) (end 152.4 88.207) (width 0.4) (layer "F.Cu") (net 25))
 (segment (start 129.732 87.544) (end 151.444 87.544) (width 0.4) (layer "F.Cu") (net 25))
 (segment (start 152.4 88.207) (end 152.107 88.207) (width 0.4) (layer "F.Cu") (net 25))
 (segment (start 120.777 89.429) (end 120.502 89.154) (width 0.4) (layer "F.Cu") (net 26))
 (segment (start 121.539 92.329) (end 120.777 91.567) (width 0.4) (layer "F.Cu") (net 26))
 (segment (start 152.4 95.765) (end 158.9 95.765) (width 0.4) (layer "F.Cu") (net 26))
 (segment (start 147.786309 92.774001) (end 125.032001 92.774001) (width 0.4) (layer "F.Cu") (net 26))
 (segment (start 152.198 95.556) (end 149.733 93.091) (width 0.4) (layer "F.Cu") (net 26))
 (segment (start 125.032001 92.774001) (end 124.587 92.329) (width 0.4) (layer "F.Cu") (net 26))
 (segment (start 120.777 91.567) (end 120.777 89.429) (width 0.4) (layer "F.Cu") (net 26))
 (via (at 124.587 92.329) (size 0.6) (drill 0.3) (layers "F.Cu" "B.Cu") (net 26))
 (via (at 149.733 93.091) (size 0.6) (drill 0.3) (layers "F.Cu" "B.Cu") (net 26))
 (via (at 121.539 92.329) (size 0.6) (drill 0.3) (layers "F.Cu" "B.Cu") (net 26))
 (via (at 147.786309 92.774001) (size 0.6) (drill 0.3) (layers "F.Cu" "B.Cu") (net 26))
 (segment (start 149.416001 92.774001) (end 147.786309 92.774001) (width 0.4) (layer "B.Cu") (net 26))
 (segment (start 121.539 92.329) (end 124.587 92.329) (width 0.4) (layer "B.Cu") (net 26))
 (segment (start 149.733 93.091) (end 149.416001 92.774001) (width 0.4) (layer "B.Cu") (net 26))
 (segment (start 124.169 91.613) (end 123.742 91.186) (width 0.4) (layer "F.Cu") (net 27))
 (segment (start 148.993 92.989328) (end 147.616672 91.613) (width 0.4) (layer "F.Cu") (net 27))
 (segment (start 147.616672 91.613) (end 124.169 91.613) (width 0.4) (layer "F.Cu") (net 27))
 (segment (start 148.993 100.209) (end 148.993 92.989328) (width 0.4) (layer "F.Cu") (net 27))
 (segment (start 152.198 103.414) (end 148.993 100.209) (width 0.4) (layer "F.Cu") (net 27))
 (segment (start 152.4 103.323) (end 158.9 103.323) (width 0.4) (layer "F.Cu") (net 27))
 (via (at 123.742 91.186) (size 0.6) (drill 0.3) (layers "F.Cu" "B.Cu") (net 27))
 (segment (start 119.994 91.186) (end 117.962 89.154) (width 0.4) (layer "B.Cu") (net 27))
 (segment (start 123.742 91.186) (end 119.994 91.186) (width 0.4) (layer "B.Cu") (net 27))
 (segment (start 152.224 110.881) (end 151.726 111.379) (width 0.4) (layer "F.Cu") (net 4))
 (segment (start 152.4 110.881) (end 152.224 110.881) (width 0.4) (layer "F.Cu") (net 4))
 (segment (start 151.726 111.379) (end 141.922172 111.379) (width 0.4) (layer "F.Cu") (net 4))
 (segment (start 141.922172 111.379) (end 123.042 92.498828) (width 0.4) (layer "F.Cu") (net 4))
 (segment (start 123.042 92.498828) (end 123.042 89.154) (width 0.4) (layer "F.Cu") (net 4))
 (segment (start 158.9 110.881) (end 152.4 110.881) (width 0.4) (layer "F.Cu") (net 4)))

